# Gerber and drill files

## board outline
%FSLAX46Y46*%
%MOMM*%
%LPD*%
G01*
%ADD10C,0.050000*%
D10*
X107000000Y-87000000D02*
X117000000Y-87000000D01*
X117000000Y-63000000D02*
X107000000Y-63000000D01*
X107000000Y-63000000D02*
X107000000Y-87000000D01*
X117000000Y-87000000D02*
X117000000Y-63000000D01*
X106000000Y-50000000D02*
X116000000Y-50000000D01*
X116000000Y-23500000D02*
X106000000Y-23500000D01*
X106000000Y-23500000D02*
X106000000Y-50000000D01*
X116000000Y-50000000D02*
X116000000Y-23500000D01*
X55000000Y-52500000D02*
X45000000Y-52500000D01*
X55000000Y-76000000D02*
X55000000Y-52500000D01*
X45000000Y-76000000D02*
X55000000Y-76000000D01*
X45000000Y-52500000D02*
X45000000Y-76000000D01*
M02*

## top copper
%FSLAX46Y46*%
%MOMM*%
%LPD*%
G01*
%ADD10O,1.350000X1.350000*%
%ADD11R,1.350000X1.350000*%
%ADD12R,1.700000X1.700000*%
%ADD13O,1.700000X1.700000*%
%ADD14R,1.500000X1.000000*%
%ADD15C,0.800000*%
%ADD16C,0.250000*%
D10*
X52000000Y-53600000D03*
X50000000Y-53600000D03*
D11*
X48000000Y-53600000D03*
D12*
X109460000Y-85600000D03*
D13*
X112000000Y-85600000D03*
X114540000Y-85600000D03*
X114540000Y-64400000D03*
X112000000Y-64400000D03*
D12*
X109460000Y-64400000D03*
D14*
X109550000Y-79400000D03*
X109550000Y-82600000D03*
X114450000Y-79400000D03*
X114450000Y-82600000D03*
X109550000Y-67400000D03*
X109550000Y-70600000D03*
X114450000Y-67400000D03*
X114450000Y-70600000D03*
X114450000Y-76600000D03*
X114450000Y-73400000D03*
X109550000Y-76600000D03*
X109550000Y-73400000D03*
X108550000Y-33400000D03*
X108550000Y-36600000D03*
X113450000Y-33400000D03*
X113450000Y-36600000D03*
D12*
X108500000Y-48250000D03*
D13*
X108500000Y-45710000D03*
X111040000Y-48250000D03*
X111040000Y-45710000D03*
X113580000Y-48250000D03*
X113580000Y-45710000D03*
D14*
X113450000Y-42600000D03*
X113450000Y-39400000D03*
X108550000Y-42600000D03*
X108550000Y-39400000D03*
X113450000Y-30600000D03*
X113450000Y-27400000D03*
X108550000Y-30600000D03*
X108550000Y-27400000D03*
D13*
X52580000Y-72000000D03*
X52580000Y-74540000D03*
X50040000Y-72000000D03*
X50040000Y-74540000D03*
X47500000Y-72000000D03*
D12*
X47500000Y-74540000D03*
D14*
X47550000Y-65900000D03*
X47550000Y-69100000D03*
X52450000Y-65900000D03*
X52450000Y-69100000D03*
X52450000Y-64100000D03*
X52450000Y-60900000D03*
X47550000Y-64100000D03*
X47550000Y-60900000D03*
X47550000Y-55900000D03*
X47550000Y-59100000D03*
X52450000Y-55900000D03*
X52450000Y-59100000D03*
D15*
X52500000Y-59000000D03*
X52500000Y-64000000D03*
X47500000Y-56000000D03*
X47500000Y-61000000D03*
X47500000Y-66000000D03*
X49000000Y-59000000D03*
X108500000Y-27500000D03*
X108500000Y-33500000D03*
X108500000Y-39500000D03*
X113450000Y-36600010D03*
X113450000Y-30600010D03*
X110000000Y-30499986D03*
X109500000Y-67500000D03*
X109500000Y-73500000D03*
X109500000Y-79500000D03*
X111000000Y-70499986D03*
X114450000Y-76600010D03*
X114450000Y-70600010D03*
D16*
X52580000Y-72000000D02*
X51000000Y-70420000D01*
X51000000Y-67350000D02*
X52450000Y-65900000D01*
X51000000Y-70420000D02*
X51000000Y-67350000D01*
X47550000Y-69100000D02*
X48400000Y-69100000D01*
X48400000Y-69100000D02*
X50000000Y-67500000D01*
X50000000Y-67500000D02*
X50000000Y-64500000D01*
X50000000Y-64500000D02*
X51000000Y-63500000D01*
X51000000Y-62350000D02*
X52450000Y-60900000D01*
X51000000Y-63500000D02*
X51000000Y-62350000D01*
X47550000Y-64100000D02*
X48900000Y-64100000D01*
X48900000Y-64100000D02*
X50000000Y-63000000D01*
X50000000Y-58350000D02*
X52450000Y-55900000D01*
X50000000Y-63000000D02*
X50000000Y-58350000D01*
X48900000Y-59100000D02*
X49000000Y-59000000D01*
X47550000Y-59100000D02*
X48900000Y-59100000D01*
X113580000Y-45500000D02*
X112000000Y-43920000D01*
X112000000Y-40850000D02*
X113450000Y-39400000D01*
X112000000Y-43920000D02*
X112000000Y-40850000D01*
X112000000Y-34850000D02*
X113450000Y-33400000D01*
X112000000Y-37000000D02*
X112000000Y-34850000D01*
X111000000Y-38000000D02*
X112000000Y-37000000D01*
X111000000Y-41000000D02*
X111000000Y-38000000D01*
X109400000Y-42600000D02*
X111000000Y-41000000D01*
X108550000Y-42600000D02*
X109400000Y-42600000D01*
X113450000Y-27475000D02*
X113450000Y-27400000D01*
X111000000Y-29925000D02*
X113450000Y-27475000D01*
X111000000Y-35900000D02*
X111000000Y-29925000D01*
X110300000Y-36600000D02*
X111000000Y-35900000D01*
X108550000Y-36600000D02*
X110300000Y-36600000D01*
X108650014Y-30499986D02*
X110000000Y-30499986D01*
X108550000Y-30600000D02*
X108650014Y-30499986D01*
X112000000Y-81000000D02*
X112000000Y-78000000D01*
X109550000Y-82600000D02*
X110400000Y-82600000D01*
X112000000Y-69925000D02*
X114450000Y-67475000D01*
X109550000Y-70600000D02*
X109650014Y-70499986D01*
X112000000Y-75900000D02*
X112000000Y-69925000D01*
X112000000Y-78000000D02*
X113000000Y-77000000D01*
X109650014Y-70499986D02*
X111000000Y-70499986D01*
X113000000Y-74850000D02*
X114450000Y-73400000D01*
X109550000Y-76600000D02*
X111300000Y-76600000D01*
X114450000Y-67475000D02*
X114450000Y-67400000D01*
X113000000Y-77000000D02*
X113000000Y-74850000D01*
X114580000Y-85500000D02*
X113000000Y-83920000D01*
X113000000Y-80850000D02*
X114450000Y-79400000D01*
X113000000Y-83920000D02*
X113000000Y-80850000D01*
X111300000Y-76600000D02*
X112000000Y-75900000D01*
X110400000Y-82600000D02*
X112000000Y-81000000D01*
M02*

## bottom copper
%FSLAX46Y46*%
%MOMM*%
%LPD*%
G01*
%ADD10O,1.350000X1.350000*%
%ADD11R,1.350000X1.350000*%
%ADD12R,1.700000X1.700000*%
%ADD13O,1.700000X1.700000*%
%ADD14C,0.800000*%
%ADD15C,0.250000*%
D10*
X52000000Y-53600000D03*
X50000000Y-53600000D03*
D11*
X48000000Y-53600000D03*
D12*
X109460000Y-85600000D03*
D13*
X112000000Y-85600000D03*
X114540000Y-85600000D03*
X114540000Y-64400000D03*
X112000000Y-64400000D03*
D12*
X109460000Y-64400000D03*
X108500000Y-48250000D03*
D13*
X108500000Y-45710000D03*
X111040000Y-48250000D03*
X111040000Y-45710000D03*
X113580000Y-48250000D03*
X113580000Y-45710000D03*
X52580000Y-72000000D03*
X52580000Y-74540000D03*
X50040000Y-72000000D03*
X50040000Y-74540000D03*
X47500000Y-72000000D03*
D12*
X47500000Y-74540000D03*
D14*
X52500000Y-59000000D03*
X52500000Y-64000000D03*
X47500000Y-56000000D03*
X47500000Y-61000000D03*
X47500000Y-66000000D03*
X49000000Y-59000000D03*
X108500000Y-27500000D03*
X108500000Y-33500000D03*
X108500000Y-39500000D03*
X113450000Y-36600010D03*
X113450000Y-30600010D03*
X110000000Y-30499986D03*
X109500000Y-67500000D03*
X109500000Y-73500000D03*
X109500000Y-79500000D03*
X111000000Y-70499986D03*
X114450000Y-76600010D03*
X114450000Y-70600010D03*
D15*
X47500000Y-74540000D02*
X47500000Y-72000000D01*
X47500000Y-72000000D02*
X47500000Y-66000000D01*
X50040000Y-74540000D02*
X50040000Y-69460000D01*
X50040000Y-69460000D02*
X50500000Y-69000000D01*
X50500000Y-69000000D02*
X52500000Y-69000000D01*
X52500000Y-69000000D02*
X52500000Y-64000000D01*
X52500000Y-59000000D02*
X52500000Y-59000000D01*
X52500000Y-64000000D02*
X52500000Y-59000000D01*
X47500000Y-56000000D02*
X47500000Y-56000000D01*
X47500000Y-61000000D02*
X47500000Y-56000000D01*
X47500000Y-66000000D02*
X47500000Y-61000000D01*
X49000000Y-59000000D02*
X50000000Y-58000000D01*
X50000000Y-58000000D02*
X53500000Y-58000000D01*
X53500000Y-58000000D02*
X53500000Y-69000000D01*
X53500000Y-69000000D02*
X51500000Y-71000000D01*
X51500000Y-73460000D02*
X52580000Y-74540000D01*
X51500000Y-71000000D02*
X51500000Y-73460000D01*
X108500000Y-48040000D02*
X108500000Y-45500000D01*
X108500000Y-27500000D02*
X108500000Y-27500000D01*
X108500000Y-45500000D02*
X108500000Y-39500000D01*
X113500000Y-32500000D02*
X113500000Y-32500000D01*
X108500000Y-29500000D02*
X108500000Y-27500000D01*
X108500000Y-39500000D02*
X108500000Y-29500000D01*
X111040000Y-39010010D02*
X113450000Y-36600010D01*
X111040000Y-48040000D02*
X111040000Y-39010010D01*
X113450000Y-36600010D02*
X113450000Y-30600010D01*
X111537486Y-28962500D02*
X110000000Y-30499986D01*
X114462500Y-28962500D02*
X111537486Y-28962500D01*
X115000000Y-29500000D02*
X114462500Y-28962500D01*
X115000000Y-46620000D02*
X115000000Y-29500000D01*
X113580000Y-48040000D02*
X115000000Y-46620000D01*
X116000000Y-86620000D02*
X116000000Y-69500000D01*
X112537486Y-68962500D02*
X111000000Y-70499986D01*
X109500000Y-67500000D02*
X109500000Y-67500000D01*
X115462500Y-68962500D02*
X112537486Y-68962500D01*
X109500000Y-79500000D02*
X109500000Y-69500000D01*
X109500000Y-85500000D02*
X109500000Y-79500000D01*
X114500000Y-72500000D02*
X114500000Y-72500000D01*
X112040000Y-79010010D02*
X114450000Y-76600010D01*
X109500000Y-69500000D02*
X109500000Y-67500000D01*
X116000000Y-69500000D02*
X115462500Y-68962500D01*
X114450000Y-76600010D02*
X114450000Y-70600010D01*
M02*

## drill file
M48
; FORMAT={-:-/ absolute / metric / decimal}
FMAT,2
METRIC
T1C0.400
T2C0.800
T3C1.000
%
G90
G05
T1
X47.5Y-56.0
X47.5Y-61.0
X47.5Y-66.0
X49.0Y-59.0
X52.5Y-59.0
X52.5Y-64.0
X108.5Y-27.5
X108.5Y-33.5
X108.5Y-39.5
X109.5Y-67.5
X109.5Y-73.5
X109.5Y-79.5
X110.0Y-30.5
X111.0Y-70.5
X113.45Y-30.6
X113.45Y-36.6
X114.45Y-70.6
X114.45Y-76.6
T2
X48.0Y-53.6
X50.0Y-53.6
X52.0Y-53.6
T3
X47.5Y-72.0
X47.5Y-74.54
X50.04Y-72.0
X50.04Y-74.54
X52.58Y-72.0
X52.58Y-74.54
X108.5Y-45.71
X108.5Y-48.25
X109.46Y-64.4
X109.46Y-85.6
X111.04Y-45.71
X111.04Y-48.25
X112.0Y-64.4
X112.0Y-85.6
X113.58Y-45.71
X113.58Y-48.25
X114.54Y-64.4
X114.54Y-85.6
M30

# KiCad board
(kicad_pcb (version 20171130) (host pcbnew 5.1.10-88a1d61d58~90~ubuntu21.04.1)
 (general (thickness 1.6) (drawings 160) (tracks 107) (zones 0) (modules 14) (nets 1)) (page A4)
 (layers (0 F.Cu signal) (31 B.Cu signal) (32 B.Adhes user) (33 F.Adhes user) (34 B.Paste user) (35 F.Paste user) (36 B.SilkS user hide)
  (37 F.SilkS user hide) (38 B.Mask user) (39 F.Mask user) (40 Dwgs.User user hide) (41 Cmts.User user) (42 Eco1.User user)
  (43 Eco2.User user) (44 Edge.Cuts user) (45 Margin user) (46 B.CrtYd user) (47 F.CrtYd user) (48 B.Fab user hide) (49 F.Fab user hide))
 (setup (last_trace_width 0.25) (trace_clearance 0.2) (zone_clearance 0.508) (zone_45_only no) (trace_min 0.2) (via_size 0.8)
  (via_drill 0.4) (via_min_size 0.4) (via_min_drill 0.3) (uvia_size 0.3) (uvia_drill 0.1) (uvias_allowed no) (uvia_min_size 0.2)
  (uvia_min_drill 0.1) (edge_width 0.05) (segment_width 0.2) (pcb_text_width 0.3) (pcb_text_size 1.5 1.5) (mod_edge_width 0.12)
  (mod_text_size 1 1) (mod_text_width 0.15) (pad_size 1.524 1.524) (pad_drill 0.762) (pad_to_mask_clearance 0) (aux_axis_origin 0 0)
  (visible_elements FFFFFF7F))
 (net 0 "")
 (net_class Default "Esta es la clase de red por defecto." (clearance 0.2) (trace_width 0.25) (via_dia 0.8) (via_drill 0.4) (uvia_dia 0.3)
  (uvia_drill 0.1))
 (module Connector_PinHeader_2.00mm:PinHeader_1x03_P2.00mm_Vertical (layer F.Cu) (at 48 53.6 90)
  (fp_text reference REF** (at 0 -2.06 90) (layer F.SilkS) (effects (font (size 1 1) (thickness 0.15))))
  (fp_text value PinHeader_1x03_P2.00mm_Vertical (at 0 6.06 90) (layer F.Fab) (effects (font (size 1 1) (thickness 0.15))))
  (pad 3 thru_hole oval (at 0 4 90) (size 1.35 1.35) (drill 0.8) (layers *.Cu *.Mask))
  (pad 2 thru_hole oval (at 0 2 90) (size 1.35 1.35) (drill 0.8) (layers *.Cu *.Mask))
  (pad 1 thru_hole rect (at 0 0 90) (size 1.35 1.35) (drill 0.8) (layers *.Cu *.Mask)))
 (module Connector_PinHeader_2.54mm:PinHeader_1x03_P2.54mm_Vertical (layer F.Cu) (at 109.46 85.6 90)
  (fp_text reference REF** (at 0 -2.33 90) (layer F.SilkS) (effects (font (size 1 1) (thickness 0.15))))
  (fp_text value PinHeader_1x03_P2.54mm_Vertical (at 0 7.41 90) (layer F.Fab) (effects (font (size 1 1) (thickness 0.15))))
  (pad 1 thru_hole rect (at 0 0 90) (size 1.7 1.7) (drill 1) (layers *.Cu *.Mask))
  (pad 2 thru_hole oval (at 0 2.54 90) (size 1.7 1.7) (drill 1) (layers *.Cu *.Mask))
  (pad 3 thru_hole oval (at 0 5.08 90) (size 1.7 1.7) (drill 1) (layers *.Cu *.Mask)))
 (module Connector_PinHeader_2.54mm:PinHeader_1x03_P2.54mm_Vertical (layer F.Cu) (at 109.46 64.4 90)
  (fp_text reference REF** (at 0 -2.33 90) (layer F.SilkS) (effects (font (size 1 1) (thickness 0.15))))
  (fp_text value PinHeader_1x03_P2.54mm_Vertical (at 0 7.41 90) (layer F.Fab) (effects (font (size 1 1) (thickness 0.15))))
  (pad 3 thru_hole oval (at 0 5.08 90) (size 1.7 1.7) (drill 1) (layers *.Cu *.Mask))
  (pad 2 thru_hole oval (at 0 2.54 90) (size 1.7 1.7) (drill 1) (layers *.Cu *.Mask))
  (pad 1 thru_hole rect (at 0 0 90) (size 1.7 1.7) (drill 1) (layers *.Cu *.Mask)))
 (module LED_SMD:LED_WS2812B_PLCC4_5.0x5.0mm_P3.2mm (layer F.Cu) (at 112 81)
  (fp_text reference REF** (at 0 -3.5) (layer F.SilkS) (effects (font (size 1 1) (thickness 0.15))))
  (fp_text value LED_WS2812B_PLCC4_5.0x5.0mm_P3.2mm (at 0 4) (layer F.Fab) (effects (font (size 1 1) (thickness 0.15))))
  (pad 1 smd rect (at -2.45 -1.6) (size 1.5 1) (layers F.Cu F.Paste F.Mask))
  (pad 2 smd rect (at -2.45 1.6) (size 1.5 1) (layers F.Cu F.Paste F.Mask))
  (pad 4 smd rect (at 2.45 -1.6) (size 1.5 1) (layers F.Cu F.Paste F.Mask))
  (pad 3 smd rect (at 2.45 1.6) (size 1.5 1) (layers F.Cu F.Paste F.Mask)))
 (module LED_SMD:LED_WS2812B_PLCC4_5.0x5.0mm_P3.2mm (layer F.Cu) (at 112 69)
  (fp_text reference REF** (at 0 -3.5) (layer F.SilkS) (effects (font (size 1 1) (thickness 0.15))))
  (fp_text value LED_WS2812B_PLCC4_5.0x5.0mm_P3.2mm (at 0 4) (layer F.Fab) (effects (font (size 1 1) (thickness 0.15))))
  (pad 1 smd rect (at -2.45 -1.6) (size 1.5 1) (layers F.Cu F.Paste F.Mask))
  (pad 2 smd rect (at -2.45 1.6) (size 1.5 1) (layers F.Cu F.Paste F.Mask))
  (pad 4 smd rect (at 2.45 -1.6) (size 1.5 1) (layers F.Cu F.Paste F.Mask))
  (pad 3 smd rect (at 2.45 1.6) (size 1.5 1) (layers F.Cu F.Paste F.Mask)))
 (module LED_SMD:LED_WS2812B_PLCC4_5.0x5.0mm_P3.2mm (layer F.Cu) (at 112 75)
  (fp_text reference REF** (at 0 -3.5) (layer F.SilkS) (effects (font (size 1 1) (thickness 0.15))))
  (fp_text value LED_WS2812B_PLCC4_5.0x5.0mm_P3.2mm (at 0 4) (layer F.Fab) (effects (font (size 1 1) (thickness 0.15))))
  (pad 3 smd rect (at 2.45 1.6) (size 1.5 1) (layers F.Cu F.Paste F.Mask))
  (pad 4 smd rect (at 2.45 -1.6) (size 1.5 1) (layers F.Cu F.Paste F.Mask))
  (pad 2 smd rect (at -2.45 1.6) (size 1.5 1) (layers F.Cu F.Paste F.Mask))
  (pad 1 smd rect (at -2.45 -1.6) (size 1.5 1) (layers F.Cu F.Paste F.Mask)))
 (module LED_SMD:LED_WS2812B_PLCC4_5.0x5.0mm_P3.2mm (layer F.Cu) (at 111 35)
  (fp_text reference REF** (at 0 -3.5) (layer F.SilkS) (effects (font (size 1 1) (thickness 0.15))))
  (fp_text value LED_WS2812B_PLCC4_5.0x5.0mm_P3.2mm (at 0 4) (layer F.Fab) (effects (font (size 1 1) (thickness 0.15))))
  (pad 1 smd rect (at -2.45 -1.6) (size 1.5 1) (layers F.Cu F.Paste F.Mask))
  (pad 2 smd rect (at -2.45 1.6) (size 1.5 1) (layers F.Cu F.Paste F.Mask))
  (pad 4 smd rect (at 2.45 -1.6) (size 1.5 1) (layers F.Cu F.Paste F.Mask))
  (pad 3 smd rect (at 2.45 1.6) (size 1.5 1) (layers F.Cu F.Paste F.Mask)))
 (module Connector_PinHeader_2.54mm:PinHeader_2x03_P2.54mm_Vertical (layer F.Cu) (at 108.5 48.25 90)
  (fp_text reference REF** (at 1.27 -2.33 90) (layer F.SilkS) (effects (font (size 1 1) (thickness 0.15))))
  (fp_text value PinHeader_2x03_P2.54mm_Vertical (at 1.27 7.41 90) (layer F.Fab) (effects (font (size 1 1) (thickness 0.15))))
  (pad 1 thru_hole rect (at 0 0 90) (size 1.7 1.7) (drill 1) (layers *.Cu *.Mask))
  (pad 2 thru_hole oval (at 2.54 0 90) (size 1.7 1.7) (drill 1) (layers *.Cu *.Mask))
  (pad 3 thru_hole oval (at 0 2.54 90) (size 1.7 1.7) (drill 1) (layers *.Cu *.Mask))
  (pad 4 thru_hole oval (at 2.54 2.54 90) (size 1.7 1.7) (drill 1) (layers *.Cu *.Mask))
  (pad 5 thru_hole oval (at 0 5.08 90) (size 1.7 1.7) (drill 1) (layers *.Cu *.Mask))
  (pad 6 thru_hole oval (at 2.54 5.08 90) (size 1.7 1.7) (drill 1) (layers *.Cu *.Mask)))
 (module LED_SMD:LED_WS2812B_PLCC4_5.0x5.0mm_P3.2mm (layer F.Cu) (at 111 41)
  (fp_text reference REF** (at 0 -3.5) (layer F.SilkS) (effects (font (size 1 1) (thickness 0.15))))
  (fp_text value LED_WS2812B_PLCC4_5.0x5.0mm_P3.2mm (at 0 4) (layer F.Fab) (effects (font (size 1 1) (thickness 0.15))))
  (pad 3 smd rect (at 2.45 1.6) (size 1.5 1) (layers F.Cu F.Paste F.Mask))
  (pad 4 smd rect (at 2.45 -1.6) (size 1.5 1) (layers F.Cu F.Paste F.Mask))
  (pad 2 smd rect (at -2.45 1.6) (size 1.5 1) (layers F.Cu F.Paste F.Mask))
  (pad 1 smd rect (at -2.45 -1.6) (size 1.5 1) (layers F.Cu F.Paste F.Mask)))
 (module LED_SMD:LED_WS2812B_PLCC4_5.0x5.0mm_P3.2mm (layer F.Cu) (at 111 29)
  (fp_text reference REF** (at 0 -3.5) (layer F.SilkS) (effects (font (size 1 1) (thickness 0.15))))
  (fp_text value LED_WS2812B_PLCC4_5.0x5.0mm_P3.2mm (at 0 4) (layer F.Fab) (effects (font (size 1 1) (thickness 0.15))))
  (pad 3 smd rect (at 2.45 1.6) (size 1.5 1) (layers F.Cu F.Paste F.Mask))
  (pad 4 smd rect (at 2.45 -1.6) (size 1.5 1) (layers F.Cu F.Paste F.Mask))
  (pad 2 smd rect (at -2.45 1.6) (size 1.5 1) (layers F.Cu F.Paste F.Mask))
  (pad 1 smd rect (at -2.45 -1.6) (size 1.5 1) (layers F.Cu F.Paste F.Mask)))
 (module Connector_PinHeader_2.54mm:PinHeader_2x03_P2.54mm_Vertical (layer F.Cu) (at 47.5 74.54 90)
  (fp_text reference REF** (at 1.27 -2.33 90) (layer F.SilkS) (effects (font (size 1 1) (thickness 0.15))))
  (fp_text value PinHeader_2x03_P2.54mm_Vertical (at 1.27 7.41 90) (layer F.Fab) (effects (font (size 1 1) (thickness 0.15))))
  (pad 6 thru_hole oval (at 2.54 5.08 90) (size 1.7 1.7) (drill 1) (layers *.Cu *.Mask))
  (pad 5 thru_hole oval (at 0 5.08 90) (size 1.7 1.7) (drill 1) (layers *.Cu *.Mask))
  (pad 4 thru_hole oval (at 2.54 2.54 90) (size 1.7 1.7) (drill 1) (layers *.Cu *.Mask))
  (pad 3 thru_hole oval (at 0 2.54 90) (size 1.7 1.7) (drill 1) (layers *.Cu *.Mask))
  (pad 2 thru_hole oval (at 2.54 0 90) (size 1.7 1.7) (drill 1) (layers *.Cu *.Mask))
  (pad 1 thru_hole rect (at 0 0 90) (size 1.7 1.7) (drill 1) (layers *.Cu *.Mask)))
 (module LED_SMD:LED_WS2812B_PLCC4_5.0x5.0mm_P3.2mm (layer F.Cu) (at 50 67.5)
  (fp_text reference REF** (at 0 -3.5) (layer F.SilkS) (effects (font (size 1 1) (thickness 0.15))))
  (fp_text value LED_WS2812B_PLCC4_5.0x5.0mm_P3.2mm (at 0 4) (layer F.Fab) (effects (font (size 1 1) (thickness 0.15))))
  (pad 1 smd rect (at -2.45 -1.6) (size 1.5 1) (layers F.Cu F.Paste F.Mask))
  (pad 2 smd rect (at -2.45 1.6) (size 1.5 1) (layers F.Cu F.Paste F.Mask))
  (pad 4 smd rect (at 2.45 -1.6) (size 1.5 1) (layers F.Cu F.Paste F.Mask))
  (pad 3 smd rect (at 2.45 1.6) (size 1.5 1) (layers F.Cu F.Paste F.Mask)))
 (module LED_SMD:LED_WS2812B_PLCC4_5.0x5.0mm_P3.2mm (layer F.Cu) (at 50 62.5)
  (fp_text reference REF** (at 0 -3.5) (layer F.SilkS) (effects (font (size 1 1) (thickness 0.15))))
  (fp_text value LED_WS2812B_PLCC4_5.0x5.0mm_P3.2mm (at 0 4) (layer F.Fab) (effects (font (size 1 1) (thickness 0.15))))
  (pad 3 smd rect (at 2.45 1.6) (size 1.5 1) (layers F.Cu F.Paste F.Mask))
  (pad 4 smd rect (at 2.45 -1.6) (size 1.5 1) (layers F.Cu F.Paste F.Mask))
  (pad 2 smd rect (at -2.45 1.6) (size 1.5 1) (layers F.Cu F.Paste F.Mask))
  (pad 1 smd rect (at -2.45 -1.6) (size 1.5 1) (layers F.Cu F.Paste F.Mask)))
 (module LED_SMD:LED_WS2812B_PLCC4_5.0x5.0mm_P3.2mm (layer F.Cu) (at 50 57.5)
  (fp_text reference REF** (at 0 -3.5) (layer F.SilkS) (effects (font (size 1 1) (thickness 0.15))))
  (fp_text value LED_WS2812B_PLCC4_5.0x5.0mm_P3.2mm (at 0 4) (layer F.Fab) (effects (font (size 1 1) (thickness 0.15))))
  (pad 1 smd rect (at -2.45 -1.6) (size 1.5 1) (layers F.Cu F.Paste F.Mask))
  (pad 2 smd rect (at -2.45 1.6) (size 1.5 1) (layers F.Cu F.Paste F.Mask))
  (pad 4 smd rect (at 2.45 -1.6) (size 1.5 1) (layers F.Cu F.Paste F.Mask))
  (pad 3 smd rect (at 2.45 1.6) (size 1.5 1) (layers F.Cu F.Paste F.Mask)))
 (gr_line (start 107 87) (end 117 87) (layer Edge.Cuts) (width 0.05))
 (gr_line (start 117 63) (end 107 63) (layer Edge.Cuts) (width 0.05))
 (gr_line (start 107 63) (end 107 87) (layer Edge.Cuts) (width 0.05))
 (gr_line (start 117 87) (end 117 63) (layer Edge.Cuts) (width 0.05))
 (gr_line (start 106 50) (end 116 50) (layer Edge.Cuts) (width 0.05))
 (gr_line (start 116 23.5) (end 106 23.5) (layer Edge.Cuts) (width 0.05))
 (gr_line (start 106 23.5) (end 106 50) (layer Edge.Cuts) (width 0.05))
 (gr_line (start 116 50) (end 116 23.5) (layer Edge.Cuts) (width 0.05))
 (gr_line (start 55 52.5) (end 45 52.5) (layer Edge.Cuts) (width 0.05))
 (gr_line (start 55 76) (end 55 52.5) (layer Edge.Cuts) (width 0.05))
 (gr_line (start 45 76) (end 55 76) (layer Edge.Cuts) (width 0.05))
 (gr_line (start 45 52.5) (end 45 76) (layer Edge.Cuts) (width 0.05))
 (segment (start 47.5 74.54) (end 47.5 72) (width 0.25) (layer B.Cu) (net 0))
 (segment (start 47.5 72) (end 47.5 66) (width 0.25) (layer B.Cu) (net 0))
 (segment (start 50.04 74.54) (end 50.04 69.46) (width 0.25) (layer B.Cu) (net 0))
 (segment (start 50.04 69.46) (end 50.5 69) (width 0.25) (layer B.Cu) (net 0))
 (segment (start 50.5 69) (end 52.5 69) (width 0.25) (layer B.Cu) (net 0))
 (segment (start 52.5 69) (end 52.5 64) (width 0.25) (layer B.Cu) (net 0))
 (segment (start 52.5 59) (end 52.5 59) (width 0.25) (layer B.Cu) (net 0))
 (via (at 52.5 59) (size 0.8) (drill 0.4) (layers F.Cu B.Cu) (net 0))
 (segment (start 52.5 64) (end 52.5 59) (width 0.25) (layer B.Cu) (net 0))
 (via (at 52.5 64) (size 0.8) (drill 0.4) (layers F.Cu B.Cu) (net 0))
 (segment (start 47.5 56) (end 47.5 56) (width 0.25) (layer B.Cu) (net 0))
 (via (at 47.5 56) (size 0.8) (drill 0.4) (layers F.Cu B.Cu) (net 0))
 (segment (start 47.5 61) (end 47.5 56) (width 0.25) (layer B.Cu) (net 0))
 (via (at 47.5 61) (size 0.8) (drill 0.4) (layers F.Cu B.Cu) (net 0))
 (segment (start 47.5 66) (end 47.5 61) (width 0.25) (layer B.Cu) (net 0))
 (via (at 47.5 66) (size 0.8) (drill 0.4) (layers F.Cu B.Cu) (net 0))
 (segment (start 52.58 72) (end 51 70.42) (width 0.25) (layer F.Cu) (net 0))
 (segment (start 51 67.35) (end 52.45 65.9) (width 0.25) (layer F.Cu) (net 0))
 (segment (start 51 70.42) (end 51 67.35) (width 0.25) (layer F.Cu) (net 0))
 (segment (start 47.55 69.1) (end 48.4 69.1) (width 0.25) (layer F.Cu) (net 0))
 (segment (start 48.4 69.1) (end 50 67.5) (width 0.25) (layer F.Cu) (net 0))
 (segment (start 50 67.5) (end 50 64.5) (width 0.25) (layer F.Cu) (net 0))
 (segment (start 50 64.5) (end 51 63.5) (width 0.25) (layer F.Cu) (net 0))
 (segment (start 51 62.35) (end 52.45 60.9) (width 0.25) (layer F.Cu) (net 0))
 (segment (start 51 63.5) (end 51 62.35) (width 0.25) (layer F.Cu) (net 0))
 (segment (start 47.55 64.1) (end 48.9 64.1) (width 0.25) (layer F.Cu) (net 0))
 (segment (start 48.9 64.1) (end 50 63) (width 0.25) (layer F.Cu) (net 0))
 (segment (start 50 58.35) (end 52.45 55.9) (width 0.25) (layer F.Cu) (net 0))
 (segment (start 50 63) (end 50 58.35) (width 0.25) (layer F.Cu) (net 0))
 (via (at 49 59) (size 0.8) (drill 0.4) (layers F.Cu B.Cu) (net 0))
 (segment (start 48.9 59.1) (end 49 59) (width 0.25) (layer F.Cu) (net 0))
 (segment (start 47.55 59.1) (end 48.9 59.1) (width 0.25) (layer F.Cu) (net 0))
 (segment (start 49 59) (end 50 58) (width 0.25) (layer B.Cu) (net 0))
 (segment (start 50 58) (end 53.5 58) (width 0.25) (layer B.Cu) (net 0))
 (segment (start 53.5 58) (end 53.5 69) (width 0.25) (layer B.Cu) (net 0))
 (segment (start 53.5 69) (end 51.5 71) (width 0.25) (layer B.Cu) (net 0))
 (segment (start 51.5 73.46) (end 52.58 74.54) (width 0.25) (layer B.Cu) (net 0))
 (segment (start 51.5 71) (end 51.5 73.46) (width 0.25) (layer B.Cu) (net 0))
 (segment (start 108.5 48.04) (end 108.5 45.5) (width 0.25) (layer B.Cu) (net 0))
 (segment (start 108.5 27.5) (end 108.5 27.5) (width 0.25) (layer B.Cu) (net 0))
 (via (at 108.5 27.5) (size 0.8) (drill 0.4) (layers F.Cu B.Cu) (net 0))
 (via (at 108.5 33.5) (size 0.8) (drill 0.4) (layers F.Cu B.Cu) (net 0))
 (via (at 108.5 39.5) (size 0.8) (drill 0.4) (layers F.Cu B.Cu) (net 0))
 (segment (start 113.58 45.5) (end 112 43.92) (width 0.25) (layer F.Cu) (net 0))
 (segment (start 112 40.85) (end 113.45 39.4) (width 0.25) (layer F.Cu) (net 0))
 (segment (start 112 43.92) (end 112 40.85) (width 0.25) (layer F.Cu) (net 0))
 (segment (start 108.5 45.5) (end 108.5 39.5) (width 0.25) (layer B.Cu) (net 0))
 (segment (start 113.5 32.5) (end 113.5 32.5) (width 0.25) (layer B.Cu) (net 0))
 (segment (start 108.5 29.5) (end 108.5 27.5) (width 0.25) (layer B.Cu) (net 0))
 (segment (start 108.5 39.5) (end 108.5 29.5) (width 0.25) (layer B.Cu) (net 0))
 (segment (start 112 34.85) (end 113.45 33.4) (width 0.25) (layer F.Cu) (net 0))
 (segment (start 112 37) (end 112 34.85) (width 0.25) (layer F.Cu) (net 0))
 (segment (start 111 38) (end 112 37) (width 0.25) (layer F.Cu) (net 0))
 (segment (start 111 41) (end 111 38) (width 0.25) (layer F.Cu) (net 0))
 (segment (start 109.4 42.6) (end 111 41) (width 0.25) (layer F.Cu) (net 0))
 (segment (start 108.55 42.6) (end 109.4 42.6) (width 0.25) (layer F.Cu) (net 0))
 (segment (start 113.45 27.475) (end 113.45 27.4) (width 0.25) (layer F.Cu) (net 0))
 (segment (start 111 29.925) (end 113.45 27.475) (width 0.25) (layer F.Cu) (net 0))
 (segment (start 111 35.9) (end 111 29.925) (width 0.25) (layer F.Cu) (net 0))
 (segment (start 110.3 36.6) (end 111 35.9) (width 0.25) (layer F.Cu) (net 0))
 (segment (start 108.55 36.6) (end 110.3 36.6) (width 0.25) (layer F.Cu) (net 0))
 (via (at 113.45 36.60001) (size 0.8) (drill 0.4) (layers F.Cu B.Cu) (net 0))
 (segment (start 111.04 39.01001) (end 113.45 36.60001) (width 0.25) (layer B.Cu) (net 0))
 (segment (start 111.04 48.04) (end 111.04 39.01001) (width 0.25) (layer B.Cu) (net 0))
 (via (at 113.45 30.60001) (size 0.8) (drill 0.4) (layers F.Cu B.Cu) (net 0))
 (segment (start 113.45 36.60001) (end 113.45 30.60001) (width 0.25) (layer B.Cu) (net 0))
 (via (at 110 30.499986) (size 0.8) (drill 0.4) (layers F.Cu B.Cu) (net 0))
 (segment (start 108.650014 30.499986) (end 110 30.499986) (width 0.25) (layer F.Cu) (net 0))
 (segment (start 108.55 30.6) (end 108.650014 30.499986) (width 0.25) (layer F.Cu) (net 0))
 (segment (start 111.537486 28.9625) (end 110 30.499986) (width 0.25) (layer B.Cu) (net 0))
 (segment (start 114.4625 28.9625) (end 111.537486 28.9625) (width 0.25) (layer B.Cu) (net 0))
 (segment (start 115 29.5) (end 114.4625 28.9625) (width 0.25) (layer B.Cu) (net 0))
 (segment (start 115 46.62) (end 115 29.5) (width 0.25) (layer B.Cu) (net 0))
 (segment (start 113.58 48.04) (end 115 46.62) (width 0.25) (layer B.Cu) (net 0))
 (segment (start 112 81) (end 112 78) (width 0.25) (layer F.Cu) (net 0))
 (segment (start 109.55 82.6) (end 110.4 82.6) (width 0.25) (layer F.Cu) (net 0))
 (segment (start 116 86.62) (end 116 69.5) (width 0.25) (layer B.Cu) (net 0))
 (segment (start 112 69.925) (end 114.45 67.475) (width 0.25) (layer F.Cu) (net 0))
 (segment (start 109.55 70.6) (end 109.650014 70.499986) (width 0.25) (layer F.Cu) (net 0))
 (segment (start 112 75.9) (end 112 69.925) (width 0.25) (layer F.Cu) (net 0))
 (segment (start 112 78) (end 113 77) (width 0.25) (layer F.Cu) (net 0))
 (segment (start 112.537486 68.9625) (end 111 70.499986) (width 0.25) (layer B.Cu) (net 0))
 (segment (start 109.5 67.5) (end 109.5 67.5) (width 0.25) (layer B.Cu) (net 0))
 (segment (start 109.650014 70.499986) (end 111 70.499986) (width 0.25) (layer F.Cu) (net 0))
 (via (at 109.5 67.5) (size 0.8) (drill 0.4) (layers F.Cu B.Cu) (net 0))
 (via (at 109.5 73.5) (size 0.8) (drill 0.4) (layers F.Cu B.Cu) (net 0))
 (via (at 109.5 79.5) (size 0.8) (drill 0.4) (layers F.Cu B.Cu) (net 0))
 (segment (start 113 74.85) (end 114.45 73.4) (width 0.25) (layer F.Cu) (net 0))
 (segment (start 109.55 76.6) (end 111.3 76.6) (width 0.25) (layer F.Cu) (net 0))
 (segment (start 114.45 67.475) (end 114.45 67.4) (width 0.25) (layer F.Cu) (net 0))
 (segment (start 115.4625 68.9625) (end 112.537486 68.9625) (width 0.25) (layer B.Cu) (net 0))
 (segment (start 113 77) (end 113 74.85) (width 0.25) (layer F.Cu) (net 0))
 (via (at 111 70.499986) (size 0.8) (drill 0.4) (layers F.Cu B.Cu) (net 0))
 (segment (start 109.5 79.5) (end 109.5 69.5) (width 0.25) (layer B.Cu) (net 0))
 (segment (start 114.58 85.5) (end 113 83.92) (width 0.25) (layer F.Cu) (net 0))
 (segment (start 113 80.85) (end 114.45 79.4) (width 0.25) (layer F.Cu) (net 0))
 (segment (start 113 83.92) (end 113 80.85) (width 0.25) (layer F.Cu) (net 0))
 (segment (start 109.5 85.5) (end 109.5 79.5) (width 0.25) (layer B.Cu) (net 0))
 (segment (start 114.5 72.5) (end 114.5 72.5) (width 0.25) (layer B.Cu) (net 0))
 (via (at 114.45 76.60001) (size 0.8) (drill 0.4) (layers F.Cu B.Cu) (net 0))
 (via (at 114.45 70.60001) (size 0.8) (drill 0.4) (layers F.Cu B.Cu) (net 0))
 (segment (start 112.04 79.01001) (end 114.45 76.60001) (width 0.25) (layer B.Cu) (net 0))
 (segment (start 111.3 76.6) (end 112 75.9) (width 0.25) (layer F.Cu) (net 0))
 (segment (start 109.5 69.5) (end 109.5 67.5) (width 0.25) (layer B.Cu) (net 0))
 (segment (start 116 69.5) (end 115.4625 68.9625) (width 0.25) (layer B.Cu) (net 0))
 (segment (start 114.45 76.60001) (end 114.45 70.60001) (width 0.25) (layer B.Cu) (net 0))
 (segment (start 110.4 82.6) (end 112 81) (width 0.25) (layer F.Cu) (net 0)))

